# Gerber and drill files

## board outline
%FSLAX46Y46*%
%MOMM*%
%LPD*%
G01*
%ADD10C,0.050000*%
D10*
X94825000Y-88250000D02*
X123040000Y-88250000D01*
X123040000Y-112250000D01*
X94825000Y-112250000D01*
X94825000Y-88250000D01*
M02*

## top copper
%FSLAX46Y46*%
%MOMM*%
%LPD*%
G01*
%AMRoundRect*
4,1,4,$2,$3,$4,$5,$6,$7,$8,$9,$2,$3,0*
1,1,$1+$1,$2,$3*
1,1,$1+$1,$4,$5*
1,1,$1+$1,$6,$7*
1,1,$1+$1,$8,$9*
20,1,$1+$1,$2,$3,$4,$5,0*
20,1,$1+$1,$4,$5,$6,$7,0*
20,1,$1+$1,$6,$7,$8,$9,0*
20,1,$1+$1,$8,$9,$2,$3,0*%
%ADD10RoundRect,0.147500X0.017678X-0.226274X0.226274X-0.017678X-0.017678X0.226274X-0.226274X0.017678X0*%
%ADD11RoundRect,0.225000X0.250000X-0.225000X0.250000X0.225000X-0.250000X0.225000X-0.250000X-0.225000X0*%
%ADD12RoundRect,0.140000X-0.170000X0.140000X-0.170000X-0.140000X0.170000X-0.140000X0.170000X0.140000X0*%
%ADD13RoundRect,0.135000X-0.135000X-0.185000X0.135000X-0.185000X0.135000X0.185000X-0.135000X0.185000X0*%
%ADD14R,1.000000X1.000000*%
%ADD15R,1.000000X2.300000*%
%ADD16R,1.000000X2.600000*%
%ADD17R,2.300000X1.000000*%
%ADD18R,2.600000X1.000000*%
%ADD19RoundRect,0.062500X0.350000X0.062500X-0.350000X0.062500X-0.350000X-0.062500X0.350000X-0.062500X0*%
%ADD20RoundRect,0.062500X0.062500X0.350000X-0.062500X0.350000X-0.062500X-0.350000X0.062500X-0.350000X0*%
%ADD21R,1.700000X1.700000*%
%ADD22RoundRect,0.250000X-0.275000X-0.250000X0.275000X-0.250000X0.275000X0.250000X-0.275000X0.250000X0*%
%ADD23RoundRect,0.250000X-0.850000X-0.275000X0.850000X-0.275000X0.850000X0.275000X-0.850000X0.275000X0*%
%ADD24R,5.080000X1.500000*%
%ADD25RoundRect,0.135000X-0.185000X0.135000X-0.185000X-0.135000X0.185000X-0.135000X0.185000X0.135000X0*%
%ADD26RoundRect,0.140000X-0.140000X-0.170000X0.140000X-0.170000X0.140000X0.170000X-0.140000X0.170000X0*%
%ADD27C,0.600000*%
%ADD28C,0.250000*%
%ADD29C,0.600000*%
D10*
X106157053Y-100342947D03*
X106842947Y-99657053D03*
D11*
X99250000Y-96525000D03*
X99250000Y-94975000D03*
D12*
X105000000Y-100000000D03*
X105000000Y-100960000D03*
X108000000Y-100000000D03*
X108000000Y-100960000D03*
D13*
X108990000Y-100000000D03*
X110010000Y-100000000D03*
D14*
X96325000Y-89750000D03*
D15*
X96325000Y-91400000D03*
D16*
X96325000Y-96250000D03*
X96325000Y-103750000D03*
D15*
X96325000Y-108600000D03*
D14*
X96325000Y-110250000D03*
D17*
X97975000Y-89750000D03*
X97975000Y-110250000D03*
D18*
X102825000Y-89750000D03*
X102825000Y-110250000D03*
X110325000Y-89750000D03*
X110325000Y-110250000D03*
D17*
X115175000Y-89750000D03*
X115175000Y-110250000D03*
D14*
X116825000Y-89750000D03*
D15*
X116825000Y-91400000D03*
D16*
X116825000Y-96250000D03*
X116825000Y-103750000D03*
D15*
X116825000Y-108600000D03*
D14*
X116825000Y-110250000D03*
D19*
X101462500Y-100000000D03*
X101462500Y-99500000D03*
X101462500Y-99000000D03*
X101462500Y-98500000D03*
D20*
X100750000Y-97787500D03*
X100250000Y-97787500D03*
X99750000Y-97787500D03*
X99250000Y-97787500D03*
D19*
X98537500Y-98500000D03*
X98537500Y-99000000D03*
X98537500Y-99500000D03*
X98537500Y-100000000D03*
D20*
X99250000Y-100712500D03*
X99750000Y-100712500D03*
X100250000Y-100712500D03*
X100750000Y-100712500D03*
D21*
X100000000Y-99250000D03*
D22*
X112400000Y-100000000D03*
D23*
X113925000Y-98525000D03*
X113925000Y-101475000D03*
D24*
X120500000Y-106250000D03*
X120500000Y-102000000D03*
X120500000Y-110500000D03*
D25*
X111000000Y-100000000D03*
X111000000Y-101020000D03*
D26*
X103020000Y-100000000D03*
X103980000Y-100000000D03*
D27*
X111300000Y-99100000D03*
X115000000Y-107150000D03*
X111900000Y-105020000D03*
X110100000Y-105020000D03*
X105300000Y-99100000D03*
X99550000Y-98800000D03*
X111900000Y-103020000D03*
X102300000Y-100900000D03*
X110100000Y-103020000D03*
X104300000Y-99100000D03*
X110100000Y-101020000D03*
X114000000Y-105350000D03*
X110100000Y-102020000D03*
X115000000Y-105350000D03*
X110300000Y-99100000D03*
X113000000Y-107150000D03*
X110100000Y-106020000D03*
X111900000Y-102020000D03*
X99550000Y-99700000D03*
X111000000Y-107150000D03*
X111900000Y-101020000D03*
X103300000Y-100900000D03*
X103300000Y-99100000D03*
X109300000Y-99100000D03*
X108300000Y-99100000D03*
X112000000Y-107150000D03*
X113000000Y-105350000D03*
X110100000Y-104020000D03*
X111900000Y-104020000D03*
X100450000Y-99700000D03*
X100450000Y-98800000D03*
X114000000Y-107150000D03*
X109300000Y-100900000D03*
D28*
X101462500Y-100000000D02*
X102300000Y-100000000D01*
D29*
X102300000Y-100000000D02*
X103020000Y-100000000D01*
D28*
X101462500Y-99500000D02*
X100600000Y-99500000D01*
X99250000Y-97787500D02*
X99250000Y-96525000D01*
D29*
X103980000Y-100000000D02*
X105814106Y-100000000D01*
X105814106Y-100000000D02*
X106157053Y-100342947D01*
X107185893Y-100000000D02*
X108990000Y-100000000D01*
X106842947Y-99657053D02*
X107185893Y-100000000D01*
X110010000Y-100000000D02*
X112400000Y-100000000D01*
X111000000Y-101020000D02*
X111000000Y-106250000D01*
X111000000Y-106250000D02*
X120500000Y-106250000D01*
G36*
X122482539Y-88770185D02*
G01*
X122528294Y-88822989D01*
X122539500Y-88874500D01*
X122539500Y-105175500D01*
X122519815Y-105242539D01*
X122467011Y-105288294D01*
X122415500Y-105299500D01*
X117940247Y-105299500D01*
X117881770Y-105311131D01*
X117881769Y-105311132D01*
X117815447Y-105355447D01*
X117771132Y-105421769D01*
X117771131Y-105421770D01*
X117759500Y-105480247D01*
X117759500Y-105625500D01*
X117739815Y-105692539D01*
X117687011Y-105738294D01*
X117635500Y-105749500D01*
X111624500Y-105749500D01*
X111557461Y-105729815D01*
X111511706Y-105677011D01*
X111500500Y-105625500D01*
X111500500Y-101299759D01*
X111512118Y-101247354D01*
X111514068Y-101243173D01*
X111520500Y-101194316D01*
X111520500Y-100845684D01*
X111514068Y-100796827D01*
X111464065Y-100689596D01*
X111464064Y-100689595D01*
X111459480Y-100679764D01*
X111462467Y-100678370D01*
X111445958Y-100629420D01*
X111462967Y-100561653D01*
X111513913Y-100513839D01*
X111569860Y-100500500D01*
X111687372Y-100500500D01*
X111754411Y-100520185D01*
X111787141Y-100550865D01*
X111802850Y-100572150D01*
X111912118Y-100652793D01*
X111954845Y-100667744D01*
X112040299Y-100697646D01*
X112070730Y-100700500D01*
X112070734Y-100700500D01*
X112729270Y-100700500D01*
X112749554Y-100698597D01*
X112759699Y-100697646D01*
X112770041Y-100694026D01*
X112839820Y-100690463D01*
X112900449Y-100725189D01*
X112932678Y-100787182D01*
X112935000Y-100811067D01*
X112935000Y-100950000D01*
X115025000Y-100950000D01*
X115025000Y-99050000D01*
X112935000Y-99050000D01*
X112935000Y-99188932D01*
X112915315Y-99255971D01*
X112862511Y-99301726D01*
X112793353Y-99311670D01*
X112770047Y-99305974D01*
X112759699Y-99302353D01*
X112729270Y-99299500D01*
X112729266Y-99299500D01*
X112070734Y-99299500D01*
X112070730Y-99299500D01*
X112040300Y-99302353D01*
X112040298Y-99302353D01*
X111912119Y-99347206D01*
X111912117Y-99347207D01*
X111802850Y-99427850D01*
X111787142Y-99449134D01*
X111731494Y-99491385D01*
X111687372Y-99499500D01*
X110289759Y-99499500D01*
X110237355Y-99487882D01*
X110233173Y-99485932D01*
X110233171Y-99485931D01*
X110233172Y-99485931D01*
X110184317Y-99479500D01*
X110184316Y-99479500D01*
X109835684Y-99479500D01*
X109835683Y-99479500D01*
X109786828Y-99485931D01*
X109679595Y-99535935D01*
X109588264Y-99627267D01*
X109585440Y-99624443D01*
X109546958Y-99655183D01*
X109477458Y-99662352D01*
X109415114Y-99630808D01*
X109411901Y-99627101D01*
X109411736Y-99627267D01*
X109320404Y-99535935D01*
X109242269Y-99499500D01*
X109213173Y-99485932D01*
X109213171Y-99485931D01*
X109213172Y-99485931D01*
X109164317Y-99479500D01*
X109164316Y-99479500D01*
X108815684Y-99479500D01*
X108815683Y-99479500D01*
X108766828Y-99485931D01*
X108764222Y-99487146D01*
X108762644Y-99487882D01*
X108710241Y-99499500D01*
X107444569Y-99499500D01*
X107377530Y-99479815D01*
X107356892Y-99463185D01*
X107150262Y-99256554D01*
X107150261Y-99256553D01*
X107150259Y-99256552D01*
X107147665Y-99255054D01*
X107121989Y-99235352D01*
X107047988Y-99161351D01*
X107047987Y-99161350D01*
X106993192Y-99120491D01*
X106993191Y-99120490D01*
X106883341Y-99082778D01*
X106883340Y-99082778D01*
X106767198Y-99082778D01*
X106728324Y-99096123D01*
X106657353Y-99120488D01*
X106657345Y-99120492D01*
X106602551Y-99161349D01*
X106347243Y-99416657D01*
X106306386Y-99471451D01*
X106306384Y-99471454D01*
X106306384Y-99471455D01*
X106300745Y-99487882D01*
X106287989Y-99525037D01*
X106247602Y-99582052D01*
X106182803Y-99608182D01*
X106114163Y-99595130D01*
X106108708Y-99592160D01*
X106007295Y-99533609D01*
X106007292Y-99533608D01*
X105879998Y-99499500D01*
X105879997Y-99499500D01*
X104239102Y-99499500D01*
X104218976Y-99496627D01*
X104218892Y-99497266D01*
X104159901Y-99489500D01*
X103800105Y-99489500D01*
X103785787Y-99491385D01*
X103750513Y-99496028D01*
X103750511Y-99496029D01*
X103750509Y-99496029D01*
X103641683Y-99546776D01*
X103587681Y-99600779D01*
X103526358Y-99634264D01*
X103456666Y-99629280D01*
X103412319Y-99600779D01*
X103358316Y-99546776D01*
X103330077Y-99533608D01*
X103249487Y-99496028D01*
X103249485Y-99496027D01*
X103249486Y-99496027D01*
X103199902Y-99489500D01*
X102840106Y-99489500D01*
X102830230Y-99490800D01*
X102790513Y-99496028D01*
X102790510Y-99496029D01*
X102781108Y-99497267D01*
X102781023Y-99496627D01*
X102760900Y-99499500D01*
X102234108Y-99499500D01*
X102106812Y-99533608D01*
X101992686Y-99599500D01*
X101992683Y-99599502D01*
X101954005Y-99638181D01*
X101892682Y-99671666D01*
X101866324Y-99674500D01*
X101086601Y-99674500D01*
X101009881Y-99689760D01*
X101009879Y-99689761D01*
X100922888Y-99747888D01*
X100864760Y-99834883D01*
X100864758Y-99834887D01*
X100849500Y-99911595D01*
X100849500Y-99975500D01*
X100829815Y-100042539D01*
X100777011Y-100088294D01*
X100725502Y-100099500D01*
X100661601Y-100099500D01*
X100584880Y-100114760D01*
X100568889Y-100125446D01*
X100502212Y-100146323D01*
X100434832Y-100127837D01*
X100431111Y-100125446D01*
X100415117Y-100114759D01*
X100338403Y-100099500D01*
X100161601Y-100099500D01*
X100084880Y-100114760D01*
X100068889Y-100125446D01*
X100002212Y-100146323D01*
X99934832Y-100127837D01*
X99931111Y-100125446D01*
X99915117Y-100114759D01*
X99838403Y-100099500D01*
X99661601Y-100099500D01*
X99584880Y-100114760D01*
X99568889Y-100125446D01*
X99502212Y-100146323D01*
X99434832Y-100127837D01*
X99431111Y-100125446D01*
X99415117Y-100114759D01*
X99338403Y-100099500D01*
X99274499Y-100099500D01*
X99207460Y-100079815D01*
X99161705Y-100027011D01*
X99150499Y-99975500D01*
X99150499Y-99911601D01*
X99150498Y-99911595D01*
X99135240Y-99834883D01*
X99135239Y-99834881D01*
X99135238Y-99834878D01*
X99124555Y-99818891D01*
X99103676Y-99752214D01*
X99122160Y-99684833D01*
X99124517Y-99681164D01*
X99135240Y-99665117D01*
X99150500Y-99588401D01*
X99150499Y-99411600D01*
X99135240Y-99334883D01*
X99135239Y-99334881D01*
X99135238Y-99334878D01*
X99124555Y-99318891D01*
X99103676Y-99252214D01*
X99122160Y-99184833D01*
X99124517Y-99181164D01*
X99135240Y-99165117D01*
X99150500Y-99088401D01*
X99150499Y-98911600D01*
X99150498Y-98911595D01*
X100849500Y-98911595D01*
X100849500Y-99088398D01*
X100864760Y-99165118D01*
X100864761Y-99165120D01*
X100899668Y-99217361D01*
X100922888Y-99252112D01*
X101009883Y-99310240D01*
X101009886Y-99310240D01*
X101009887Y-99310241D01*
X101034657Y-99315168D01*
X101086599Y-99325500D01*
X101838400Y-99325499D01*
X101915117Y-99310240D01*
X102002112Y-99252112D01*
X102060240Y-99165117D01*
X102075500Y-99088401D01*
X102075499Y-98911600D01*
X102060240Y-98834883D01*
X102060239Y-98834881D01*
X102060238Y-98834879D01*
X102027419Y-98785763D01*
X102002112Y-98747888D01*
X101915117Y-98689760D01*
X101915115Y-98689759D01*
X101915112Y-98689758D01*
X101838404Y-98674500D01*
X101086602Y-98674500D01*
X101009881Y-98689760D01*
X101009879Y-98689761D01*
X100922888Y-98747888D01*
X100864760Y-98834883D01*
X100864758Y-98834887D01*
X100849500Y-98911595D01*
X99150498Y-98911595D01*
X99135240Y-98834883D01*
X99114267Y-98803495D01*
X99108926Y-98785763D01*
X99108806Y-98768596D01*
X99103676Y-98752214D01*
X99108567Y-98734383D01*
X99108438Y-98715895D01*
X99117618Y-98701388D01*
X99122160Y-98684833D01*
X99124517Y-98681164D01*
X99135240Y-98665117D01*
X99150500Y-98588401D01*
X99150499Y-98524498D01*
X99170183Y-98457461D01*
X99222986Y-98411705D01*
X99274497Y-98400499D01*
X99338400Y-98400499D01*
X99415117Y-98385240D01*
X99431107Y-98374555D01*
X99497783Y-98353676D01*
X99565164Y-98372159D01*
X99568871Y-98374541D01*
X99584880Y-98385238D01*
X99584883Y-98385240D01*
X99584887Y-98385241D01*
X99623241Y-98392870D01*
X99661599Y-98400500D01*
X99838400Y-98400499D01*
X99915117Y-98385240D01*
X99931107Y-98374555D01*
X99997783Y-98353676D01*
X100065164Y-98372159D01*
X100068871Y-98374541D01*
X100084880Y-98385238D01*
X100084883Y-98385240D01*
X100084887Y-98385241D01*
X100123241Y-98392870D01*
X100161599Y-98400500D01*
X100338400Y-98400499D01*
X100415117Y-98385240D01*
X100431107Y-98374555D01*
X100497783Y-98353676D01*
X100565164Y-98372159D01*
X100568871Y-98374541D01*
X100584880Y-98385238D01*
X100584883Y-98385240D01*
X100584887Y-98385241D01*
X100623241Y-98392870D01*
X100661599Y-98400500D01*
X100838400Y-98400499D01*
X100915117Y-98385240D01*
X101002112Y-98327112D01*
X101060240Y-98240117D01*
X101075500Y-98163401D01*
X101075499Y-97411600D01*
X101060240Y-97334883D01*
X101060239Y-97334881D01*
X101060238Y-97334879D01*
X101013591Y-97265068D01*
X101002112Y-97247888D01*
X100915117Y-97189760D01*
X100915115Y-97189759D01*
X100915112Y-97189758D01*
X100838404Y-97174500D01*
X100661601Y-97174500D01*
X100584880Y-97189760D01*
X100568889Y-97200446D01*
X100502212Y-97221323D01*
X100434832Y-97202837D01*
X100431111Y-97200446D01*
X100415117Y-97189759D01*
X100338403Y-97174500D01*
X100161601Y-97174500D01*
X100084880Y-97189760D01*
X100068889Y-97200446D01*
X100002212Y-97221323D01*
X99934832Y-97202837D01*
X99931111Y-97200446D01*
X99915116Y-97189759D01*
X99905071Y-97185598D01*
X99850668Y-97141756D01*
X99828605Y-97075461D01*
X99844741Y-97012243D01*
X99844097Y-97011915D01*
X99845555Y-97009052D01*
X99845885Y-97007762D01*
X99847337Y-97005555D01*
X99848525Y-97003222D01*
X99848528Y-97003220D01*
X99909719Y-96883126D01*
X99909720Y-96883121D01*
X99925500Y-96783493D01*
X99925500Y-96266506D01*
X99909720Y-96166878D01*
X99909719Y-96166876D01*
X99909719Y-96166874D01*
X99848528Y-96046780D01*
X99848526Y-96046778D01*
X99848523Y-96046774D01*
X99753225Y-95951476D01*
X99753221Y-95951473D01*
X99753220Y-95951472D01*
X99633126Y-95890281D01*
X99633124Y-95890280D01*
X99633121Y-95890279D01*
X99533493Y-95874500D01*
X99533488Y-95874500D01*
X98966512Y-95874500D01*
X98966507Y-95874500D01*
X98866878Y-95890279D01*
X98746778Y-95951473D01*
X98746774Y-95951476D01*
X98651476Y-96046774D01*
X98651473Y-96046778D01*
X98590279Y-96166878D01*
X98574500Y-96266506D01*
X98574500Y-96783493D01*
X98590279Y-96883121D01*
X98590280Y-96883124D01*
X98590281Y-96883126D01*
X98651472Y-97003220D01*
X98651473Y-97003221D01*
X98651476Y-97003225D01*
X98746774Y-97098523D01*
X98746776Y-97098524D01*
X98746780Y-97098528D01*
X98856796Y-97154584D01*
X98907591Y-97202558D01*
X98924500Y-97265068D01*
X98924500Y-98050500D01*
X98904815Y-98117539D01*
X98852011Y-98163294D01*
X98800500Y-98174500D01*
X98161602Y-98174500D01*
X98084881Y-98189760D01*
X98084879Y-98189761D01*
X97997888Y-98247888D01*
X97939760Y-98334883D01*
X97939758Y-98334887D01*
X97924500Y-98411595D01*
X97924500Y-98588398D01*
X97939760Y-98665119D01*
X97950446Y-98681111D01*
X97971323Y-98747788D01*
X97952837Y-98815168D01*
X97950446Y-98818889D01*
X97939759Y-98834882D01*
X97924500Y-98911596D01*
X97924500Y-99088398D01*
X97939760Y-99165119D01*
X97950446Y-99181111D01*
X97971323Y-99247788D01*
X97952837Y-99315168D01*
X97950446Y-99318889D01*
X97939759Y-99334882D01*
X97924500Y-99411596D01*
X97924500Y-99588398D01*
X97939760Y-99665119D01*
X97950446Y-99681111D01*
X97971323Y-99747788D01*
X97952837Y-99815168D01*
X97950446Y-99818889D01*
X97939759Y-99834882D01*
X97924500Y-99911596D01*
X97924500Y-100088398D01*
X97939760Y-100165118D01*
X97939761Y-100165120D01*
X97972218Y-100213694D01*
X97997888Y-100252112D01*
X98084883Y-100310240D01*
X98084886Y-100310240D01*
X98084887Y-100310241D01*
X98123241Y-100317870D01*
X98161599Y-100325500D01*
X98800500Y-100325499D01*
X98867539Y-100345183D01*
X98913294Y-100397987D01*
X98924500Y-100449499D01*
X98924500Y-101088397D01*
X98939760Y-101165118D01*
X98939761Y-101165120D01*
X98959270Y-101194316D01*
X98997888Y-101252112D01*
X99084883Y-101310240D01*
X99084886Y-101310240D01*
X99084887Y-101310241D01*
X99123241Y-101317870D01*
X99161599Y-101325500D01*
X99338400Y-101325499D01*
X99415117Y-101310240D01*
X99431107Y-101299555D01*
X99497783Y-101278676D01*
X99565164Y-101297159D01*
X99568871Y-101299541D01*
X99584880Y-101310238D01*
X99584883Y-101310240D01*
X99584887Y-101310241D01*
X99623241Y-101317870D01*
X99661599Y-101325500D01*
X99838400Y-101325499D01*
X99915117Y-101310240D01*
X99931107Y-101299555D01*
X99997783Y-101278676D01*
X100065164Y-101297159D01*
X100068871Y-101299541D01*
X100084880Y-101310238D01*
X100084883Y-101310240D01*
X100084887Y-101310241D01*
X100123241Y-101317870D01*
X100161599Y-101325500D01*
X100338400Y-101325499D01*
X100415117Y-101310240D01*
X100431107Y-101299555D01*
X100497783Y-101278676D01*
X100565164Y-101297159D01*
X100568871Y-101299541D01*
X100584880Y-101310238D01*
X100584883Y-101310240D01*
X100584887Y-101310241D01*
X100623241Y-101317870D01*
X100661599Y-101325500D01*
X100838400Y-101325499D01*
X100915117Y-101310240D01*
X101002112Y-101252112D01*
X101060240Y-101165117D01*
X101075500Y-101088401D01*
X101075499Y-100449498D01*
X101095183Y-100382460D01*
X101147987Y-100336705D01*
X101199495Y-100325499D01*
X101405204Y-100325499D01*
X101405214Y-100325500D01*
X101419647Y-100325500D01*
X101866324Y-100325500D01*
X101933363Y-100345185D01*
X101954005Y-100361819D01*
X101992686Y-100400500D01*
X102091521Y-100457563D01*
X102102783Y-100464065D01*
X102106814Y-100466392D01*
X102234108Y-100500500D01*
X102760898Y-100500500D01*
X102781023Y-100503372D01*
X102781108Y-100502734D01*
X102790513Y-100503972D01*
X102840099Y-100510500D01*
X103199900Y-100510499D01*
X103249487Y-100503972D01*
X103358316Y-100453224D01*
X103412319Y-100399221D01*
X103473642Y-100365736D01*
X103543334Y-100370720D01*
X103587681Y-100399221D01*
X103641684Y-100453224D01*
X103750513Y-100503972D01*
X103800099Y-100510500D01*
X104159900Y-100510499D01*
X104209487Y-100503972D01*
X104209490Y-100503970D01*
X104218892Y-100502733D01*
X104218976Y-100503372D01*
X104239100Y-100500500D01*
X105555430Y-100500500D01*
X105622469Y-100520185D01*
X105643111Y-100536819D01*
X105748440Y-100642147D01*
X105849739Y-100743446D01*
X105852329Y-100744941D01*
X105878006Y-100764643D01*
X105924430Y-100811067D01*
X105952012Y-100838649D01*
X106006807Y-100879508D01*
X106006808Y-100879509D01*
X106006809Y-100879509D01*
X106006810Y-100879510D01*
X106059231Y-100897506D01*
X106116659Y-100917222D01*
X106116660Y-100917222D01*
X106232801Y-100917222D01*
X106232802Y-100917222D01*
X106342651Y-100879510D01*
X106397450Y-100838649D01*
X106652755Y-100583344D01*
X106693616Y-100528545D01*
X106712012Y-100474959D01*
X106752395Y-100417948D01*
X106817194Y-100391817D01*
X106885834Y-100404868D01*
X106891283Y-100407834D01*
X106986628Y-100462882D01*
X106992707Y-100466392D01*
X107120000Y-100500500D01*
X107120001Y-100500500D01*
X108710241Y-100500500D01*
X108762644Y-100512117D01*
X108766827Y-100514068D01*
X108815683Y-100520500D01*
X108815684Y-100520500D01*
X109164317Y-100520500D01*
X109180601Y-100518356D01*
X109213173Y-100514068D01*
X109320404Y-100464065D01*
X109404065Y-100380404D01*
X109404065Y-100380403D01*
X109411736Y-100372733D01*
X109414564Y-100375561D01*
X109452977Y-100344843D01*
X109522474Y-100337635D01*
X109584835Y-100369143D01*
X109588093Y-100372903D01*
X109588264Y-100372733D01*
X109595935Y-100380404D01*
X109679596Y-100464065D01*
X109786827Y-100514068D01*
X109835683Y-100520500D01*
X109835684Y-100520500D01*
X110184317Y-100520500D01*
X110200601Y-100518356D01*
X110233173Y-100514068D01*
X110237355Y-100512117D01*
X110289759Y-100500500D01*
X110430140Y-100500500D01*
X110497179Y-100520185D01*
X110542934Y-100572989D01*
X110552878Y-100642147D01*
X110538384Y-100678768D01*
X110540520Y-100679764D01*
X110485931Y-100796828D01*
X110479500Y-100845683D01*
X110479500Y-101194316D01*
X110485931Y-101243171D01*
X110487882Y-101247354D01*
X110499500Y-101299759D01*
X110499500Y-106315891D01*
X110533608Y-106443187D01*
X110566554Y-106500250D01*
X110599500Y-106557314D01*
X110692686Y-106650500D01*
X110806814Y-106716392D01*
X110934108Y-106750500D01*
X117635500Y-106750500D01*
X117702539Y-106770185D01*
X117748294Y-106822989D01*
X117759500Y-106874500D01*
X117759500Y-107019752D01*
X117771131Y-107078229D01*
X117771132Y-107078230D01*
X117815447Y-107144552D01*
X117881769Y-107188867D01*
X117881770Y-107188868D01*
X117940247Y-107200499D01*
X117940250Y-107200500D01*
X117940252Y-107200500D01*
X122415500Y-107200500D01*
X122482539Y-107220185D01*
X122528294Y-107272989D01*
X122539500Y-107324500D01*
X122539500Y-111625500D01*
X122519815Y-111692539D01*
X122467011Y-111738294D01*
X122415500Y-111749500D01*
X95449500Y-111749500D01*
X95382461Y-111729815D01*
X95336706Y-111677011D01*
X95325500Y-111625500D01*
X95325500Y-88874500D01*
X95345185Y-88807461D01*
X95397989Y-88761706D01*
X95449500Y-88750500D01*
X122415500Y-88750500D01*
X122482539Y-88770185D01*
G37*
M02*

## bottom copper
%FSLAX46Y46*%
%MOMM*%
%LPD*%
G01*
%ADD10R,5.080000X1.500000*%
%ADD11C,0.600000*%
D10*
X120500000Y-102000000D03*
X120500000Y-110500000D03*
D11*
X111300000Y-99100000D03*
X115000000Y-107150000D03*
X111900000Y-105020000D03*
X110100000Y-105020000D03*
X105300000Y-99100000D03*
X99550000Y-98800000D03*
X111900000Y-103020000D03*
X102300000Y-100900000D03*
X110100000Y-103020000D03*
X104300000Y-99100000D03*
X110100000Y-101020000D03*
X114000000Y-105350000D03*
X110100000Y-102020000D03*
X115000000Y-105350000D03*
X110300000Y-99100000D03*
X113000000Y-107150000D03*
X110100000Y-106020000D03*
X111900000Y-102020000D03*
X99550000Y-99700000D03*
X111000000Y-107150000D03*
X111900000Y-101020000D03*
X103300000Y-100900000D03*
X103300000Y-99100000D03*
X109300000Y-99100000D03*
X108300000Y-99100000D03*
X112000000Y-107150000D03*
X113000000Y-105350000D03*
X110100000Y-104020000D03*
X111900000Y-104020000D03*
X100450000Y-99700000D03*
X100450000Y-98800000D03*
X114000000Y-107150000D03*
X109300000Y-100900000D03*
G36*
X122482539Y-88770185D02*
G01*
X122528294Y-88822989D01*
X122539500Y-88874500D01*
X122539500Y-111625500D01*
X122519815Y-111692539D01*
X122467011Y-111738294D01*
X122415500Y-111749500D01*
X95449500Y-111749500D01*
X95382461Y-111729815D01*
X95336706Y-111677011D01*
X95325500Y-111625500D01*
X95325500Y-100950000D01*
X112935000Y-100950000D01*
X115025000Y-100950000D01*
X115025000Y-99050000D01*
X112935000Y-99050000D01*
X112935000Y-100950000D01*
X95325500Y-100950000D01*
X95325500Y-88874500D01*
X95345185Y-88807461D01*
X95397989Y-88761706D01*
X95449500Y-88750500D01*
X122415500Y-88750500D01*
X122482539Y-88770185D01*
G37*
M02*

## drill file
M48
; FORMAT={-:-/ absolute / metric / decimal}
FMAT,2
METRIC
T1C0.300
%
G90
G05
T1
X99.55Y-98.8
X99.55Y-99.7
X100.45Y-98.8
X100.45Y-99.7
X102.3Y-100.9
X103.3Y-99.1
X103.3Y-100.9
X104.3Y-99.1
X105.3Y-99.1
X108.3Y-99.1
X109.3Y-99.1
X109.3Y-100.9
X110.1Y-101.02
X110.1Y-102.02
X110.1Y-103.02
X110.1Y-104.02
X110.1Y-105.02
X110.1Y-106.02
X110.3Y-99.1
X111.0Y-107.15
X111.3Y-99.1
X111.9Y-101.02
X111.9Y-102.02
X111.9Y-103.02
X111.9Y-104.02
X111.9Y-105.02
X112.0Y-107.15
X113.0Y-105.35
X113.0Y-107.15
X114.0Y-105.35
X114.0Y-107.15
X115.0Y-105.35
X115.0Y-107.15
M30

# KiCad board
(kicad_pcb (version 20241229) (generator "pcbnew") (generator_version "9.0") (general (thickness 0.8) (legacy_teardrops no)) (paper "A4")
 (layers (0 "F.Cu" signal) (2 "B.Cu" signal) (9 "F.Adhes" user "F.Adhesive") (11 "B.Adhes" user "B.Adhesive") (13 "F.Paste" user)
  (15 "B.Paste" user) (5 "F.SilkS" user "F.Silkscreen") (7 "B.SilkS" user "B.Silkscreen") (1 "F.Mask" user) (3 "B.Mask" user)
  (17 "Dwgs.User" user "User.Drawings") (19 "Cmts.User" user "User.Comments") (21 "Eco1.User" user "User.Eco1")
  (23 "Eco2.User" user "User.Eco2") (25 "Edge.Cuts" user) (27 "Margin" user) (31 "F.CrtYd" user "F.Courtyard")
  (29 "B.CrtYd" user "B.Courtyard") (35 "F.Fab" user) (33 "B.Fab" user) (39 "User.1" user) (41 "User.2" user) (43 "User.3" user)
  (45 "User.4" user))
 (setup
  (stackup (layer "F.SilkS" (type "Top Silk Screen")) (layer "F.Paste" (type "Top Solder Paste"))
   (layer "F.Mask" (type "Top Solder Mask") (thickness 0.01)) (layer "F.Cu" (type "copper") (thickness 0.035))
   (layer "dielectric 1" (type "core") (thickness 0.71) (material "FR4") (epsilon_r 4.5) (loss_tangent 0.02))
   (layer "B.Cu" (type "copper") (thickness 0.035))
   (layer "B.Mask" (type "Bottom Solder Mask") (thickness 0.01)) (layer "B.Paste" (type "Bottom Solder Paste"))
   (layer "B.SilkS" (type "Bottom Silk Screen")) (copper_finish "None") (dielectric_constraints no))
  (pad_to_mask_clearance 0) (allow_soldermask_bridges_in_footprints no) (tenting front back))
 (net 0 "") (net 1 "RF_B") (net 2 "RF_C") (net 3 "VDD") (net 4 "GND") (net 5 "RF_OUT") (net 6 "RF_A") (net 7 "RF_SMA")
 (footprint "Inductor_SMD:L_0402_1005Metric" (layer "F.Cu") (at 106.5 100 45)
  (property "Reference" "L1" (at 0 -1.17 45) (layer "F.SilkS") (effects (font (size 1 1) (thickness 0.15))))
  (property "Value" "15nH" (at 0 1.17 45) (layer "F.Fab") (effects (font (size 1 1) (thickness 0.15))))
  (pad "1" smd roundrect (at -0.485 0 45) (size 0.59 0.64) (layers "F.Cu" "F.Mask" "F.Paste") (roundrect_rratio 0.25) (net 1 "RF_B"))
  (pad "2" smd roundrect (at 0.485 0 45) (size 0.59 0.64) (layers "F.Cu" "F.Mask" "F.Paste") (roundrect_rratio 0.25) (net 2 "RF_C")))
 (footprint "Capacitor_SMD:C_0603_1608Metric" (layer "F.Cu") (at 99.25 95.75 90)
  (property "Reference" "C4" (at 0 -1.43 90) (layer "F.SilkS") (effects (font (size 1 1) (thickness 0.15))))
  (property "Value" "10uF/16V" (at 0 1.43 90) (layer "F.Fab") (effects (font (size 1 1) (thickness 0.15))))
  (pad "1" smd roundrect (at -0.775 0 90) (size 0.9 0.95) (layers "F.Cu" "F.Mask" "F.Paste") (roundrect_rratio 0.25) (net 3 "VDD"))
  (pad "2" smd roundrect (at 0.775 0 90) (size 0.9 0.95) (layers "F.Cu" "F.Mask" "F.Paste") (roundrect_rratio 0.25) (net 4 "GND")))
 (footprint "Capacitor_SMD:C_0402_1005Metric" (layer "F.Cu") (at 105 100.48 -90)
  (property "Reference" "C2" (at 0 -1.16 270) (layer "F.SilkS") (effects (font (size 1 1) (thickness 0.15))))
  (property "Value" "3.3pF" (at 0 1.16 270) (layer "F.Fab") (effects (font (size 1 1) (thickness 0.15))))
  (pad "1" smd roundrect (at -0.48 0 270) (size 0.56 0.62) (layers "F.Cu" "F.Mask" "F.Paste") (roundrect_rratio 0.25) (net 1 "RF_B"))
  (pad "2" smd roundrect (at 0.48 0 270) (size 0.56 0.62) (layers "F.Cu" "F.Mask" "F.Paste") (roundrect_rratio 0.25) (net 4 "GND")))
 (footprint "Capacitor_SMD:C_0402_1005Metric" (layer "F.Cu") (at 108 100.48 -90)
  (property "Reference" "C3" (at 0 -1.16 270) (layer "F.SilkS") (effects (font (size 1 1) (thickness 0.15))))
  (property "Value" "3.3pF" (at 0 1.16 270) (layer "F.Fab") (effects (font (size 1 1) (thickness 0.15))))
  (pad "1" smd roundrect (at -0.48 0 270) (size 0.56 0.62) (layers "F.Cu" "F.Mask" "F.Paste") (roundrect_rratio 0.25) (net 2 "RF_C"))
  (pad "2" smd roundrect (at 0.48 0 270) (size 0.56 0.62) (layers "F.Cu" "F.Mask" "F.Paste") (roundrect_rratio 0.25) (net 4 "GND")))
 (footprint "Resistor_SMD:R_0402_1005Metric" (layer "F.Cu") (at 109.5 100)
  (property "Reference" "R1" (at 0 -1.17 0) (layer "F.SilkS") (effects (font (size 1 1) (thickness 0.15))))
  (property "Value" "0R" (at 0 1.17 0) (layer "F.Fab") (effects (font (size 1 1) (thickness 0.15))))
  (pad "1" smd roundrect (at -0.51 0) (size 0.54 0.64) (layers "F.Cu" "F.Mask" "F.Paste") (roundrect_rratio 0.25) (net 2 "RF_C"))
  (pad "2" smd roundrect (at 0.51 0) (size 0.54 0.64) (layers "F.Cu" "F.Mask" "F.Paste") (roundrect_rratio 0.25) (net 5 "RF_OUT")))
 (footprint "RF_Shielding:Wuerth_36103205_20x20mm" (layer "F.Cu") (at 106.575 100)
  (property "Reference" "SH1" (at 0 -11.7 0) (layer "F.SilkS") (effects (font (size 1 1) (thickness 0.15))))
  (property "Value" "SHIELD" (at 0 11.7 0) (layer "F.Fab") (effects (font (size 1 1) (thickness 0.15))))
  (pad "1" smd rect (at -10.25 -10.25) (size 1 1) (layers "F.Cu" "F.Mask" "F.Paste") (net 4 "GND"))
  (pad "1" smd rect (at -10.25 -8.6) (size 1 2.3) (layers "F.Cu" "F.Mask" "F.Paste") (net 4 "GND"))
  (pad "1" smd rect (at -10.25 -3.75) (size 1 2.6) (layers "F.Cu" "F.Mask" "F.Paste") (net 4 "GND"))
  (pad "1" smd rect (at -10.25 3.75) (size 1 2.6) (layers "F.Cu" "F.Mask" "F.Paste") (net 4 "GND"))
  (pad "1" smd rect (at -10.25 8.6) (size 1 2.3) (layers "F.Cu" "F.Mask" "F.Paste") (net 4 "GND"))
  (pad "1" smd rect (at -10.25 10.25) (size 1 1) (layers "F.Cu" "F.Mask" "F.Paste") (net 4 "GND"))
  (pad "1" smd rect (at -8.6 -10.25) (size 2.3 1) (layers "F.Cu" "F.Mask" "F.Paste") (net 4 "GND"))
  (pad "1" smd rect (at -8.6 10.25) (size 2.3 1) (layers "F.Cu" "F.Mask" "F.Paste") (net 4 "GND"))
  (pad "1" smd rect (at -3.75 -10.25) (size 2.6 1) (layers "F.Cu" "F.Mask" "F.Paste") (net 4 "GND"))
  (pad "1" smd rect (at -3.75 10.25) (size 2.6 1) (layers "F.Cu" "F.Mask" "F.Paste") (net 4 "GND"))
  (pad "1" smd rect (at 3.75 -10.25) (size 2.6 1) (layers "F.Cu" "F.Mask" "F.Paste") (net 4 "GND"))
  (pad "1" smd rect (at 3.75 10.25) (size 2.6 1) (layers "F.Cu" "F.Mask" "F.Paste") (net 4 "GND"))
  (pad "1" smd rect (at 8.6 -10.25) (size 2.3 1) (layers "F.Cu" "F.Mask" "F.Paste") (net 4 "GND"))
  (pad "1" smd rect (at 8.6 10.25) (size 2.3 1) (layers "F.Cu" "F.Mask" "F.Paste") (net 4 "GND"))
  (pad "1" smd rect (at 10.25 -10.25) (size 1 1) (layers "F.Cu" "F.Mask" "F.Paste") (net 4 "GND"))
  (pad "1" smd rect (at 10.25 -8.6) (size 1 2.3) (layers "F.Cu" "F.Mask" "F.Paste") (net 4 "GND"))
  (pad "1" smd rect (at 10.25 -3.75) (size 1 2.6) (layers "F.Cu" "F.Mask" "F.Paste") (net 4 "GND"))
  (pad "1" smd rect (at 10.25 3.75) (size 1 2.6) (layers "F.Cu" "F.Mask" "F.Paste") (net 4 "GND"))
  (pad "1" smd rect (at 10.25 8.6) (size 1 2.3) (layers "F.Cu" "F.Mask" "F.Paste") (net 4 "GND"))
  (pad "1" smd rect (at 10.25 10.25) (size 1 1) (layers "F.Cu" "F.Mask" "F.Paste") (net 4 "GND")))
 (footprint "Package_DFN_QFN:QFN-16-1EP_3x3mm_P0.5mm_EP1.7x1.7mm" (layer "F.Cu") (at 100 99.25 180)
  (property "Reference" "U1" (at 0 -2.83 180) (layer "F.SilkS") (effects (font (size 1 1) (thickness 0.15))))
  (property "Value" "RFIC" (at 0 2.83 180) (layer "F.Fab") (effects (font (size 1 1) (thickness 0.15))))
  (pad "" smd roundrect (at -0.425 -0.425 180) (size 0.69 0.69) (layers "F.Paste") (roundrect_rratio 0.25))
  (pad "" smd roundrect (at -0.425 0.425 180) (size 0.69 0.69) (layers "F.Paste") (roundrect_rratio 0.25))
  (pad "" smd roundrect (at 0.425 -0.425 180) (size 0.69 0.69) (layers "F.Paste") (roundrect_rratio 0.25))
  (pad "" smd roundrect (at 0.425 0.425 180) (size 0.69 0.69) (layers "F.Paste") (roundrect_rratio 0.25))
  (pad "1" smd roundrect (at -1.4625 -0.75 180) (size 0.825 0.25) (layers "F.Cu" "F.Mask" "F.Paste") (roundrect_rratio 0.25) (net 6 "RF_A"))
  (pad "2" smd roundrect (at -1.4625 -0.25 180) (size 0.825 0.25) (layers "F.Cu" "F.Mask" "F.Paste") (roundrect_rratio 0.25) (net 4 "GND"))
  (pad "3" smd roundrect (at -1.4625 0.25 180) (size 0.825 0.25) (layers "F.Cu" "F.Mask" "F.Paste") (roundrect_rratio 0.25))
  (pad "4" smd roundrect (at -1.4625 0.75 180) (size 0.825 0.25) (layers "F.Cu" "F.Mask" "F.Paste") (roundrect_rratio 0.25) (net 4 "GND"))
  (pad "5" smd roundrect (at -0.75 1.4625 180) (size 0.25 0.825) (layers "F.Cu" "F.Mask" "F.Paste") (roundrect_rratio 0.25))
  (pad "6" smd roundrect (at -0.25 1.4625 180) (size 0.25 0.825) (layers "F.Cu" "F.Mask" "F.Paste") (roundrect_rratio 0.25))
  (pad "7" smd roundrect (at 0.25 1.4625 180) (size 0.25 0.825) (layers "F.Cu" "F.Mask" "F.Paste") (roundrect_rratio 0.25))
  (pad "8" smd roundrect (at 0.75 1.4625 180) (size 0.25 0.825) (layers "F.Cu" "F.Mask" "F.Paste") (roundrect_rratio 0.25) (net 3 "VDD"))
  (pad "9" smd roundrect (at 1.4625 0.75 180) (size 0.825 0.25) (layers "F.Cu" "F.Mask" "F.Paste") (roundrect_rratio 0.25))
  (pad "10" smd roundrect (at 1.4625 0.25 180) (size 0.825 0.25) (layers "F.Cu" "F.Mask" "F.Paste") (roundrect_rratio 0.25))
  (pad "11" smd roundrect (at 1.4625 -0.25 180) (size 0.825 0.25) (layers "F.Cu" "F.Mask" "F.Paste") (roundrect_rratio 0.25))
  (pad "12" smd roundrect (at 1.4625 -0.75 180) (size 0.825 0.25) (layers "F.Cu" "F.Mask" "F.Paste") (roundrect_rratio 0.25))
  (pad "13" smd roundrect (at 0.75 -1.4625 180) (size 0.25 0.825) (layers "F.Cu" "F.Mask" "F.Paste") (roundrect_rratio 0.25))
  (pad "14" smd roundrect (at 0.25 -1.4625 180) (size 0.25 0.825) (layers "F.Cu" "F.Mask" "F.Paste") (roundrect_rratio 0.25))
  (pad "15" smd roundrect (at -0.25 -1.4625 180) (size 0.25 0.825) (layers "F.Cu" "F.Mask" "F.Paste") (roundrect_rratio 0.25))
  (pad "16" smd roundrect (at -0.75 -1.4625 180) (size 0.25 0.825) (layers "F.Cu" "F.Mask" "F.Paste") (roundrect_rratio 0.25))
  (pad "17" smd rect (at 0 0 180) (size 1.7 1.7) (layers "F.Cu" "F.Mask") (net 4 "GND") (zone_connect 2)))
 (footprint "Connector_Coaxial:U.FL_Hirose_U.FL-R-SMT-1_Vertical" (layer "F.Cu") (at 113.45 100)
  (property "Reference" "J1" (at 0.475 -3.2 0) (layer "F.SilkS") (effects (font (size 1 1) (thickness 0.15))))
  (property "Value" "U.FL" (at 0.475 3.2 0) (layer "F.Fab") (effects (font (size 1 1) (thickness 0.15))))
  (pad "1" smd roundrect (at -1.05 0) (size 1.05 1) (layers "F.Cu" "F.Mask" "F.Paste") (roundrect_rratio 0.25) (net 5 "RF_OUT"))
  (pad "2" smd roundrect (at 0.475 -1.475) (size 2.2 1.05) (layers "F.Cu" "F.Mask" "F.Paste") (roundrect_rratio 0.2380952381) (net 4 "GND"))
  (pad "2" smd roundrect (at 0.475 1.475) (size 2.2 1.05) (layers "F.Cu" "F.Mask" "F.Paste") (roundrect_rratio 0.2380952381) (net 4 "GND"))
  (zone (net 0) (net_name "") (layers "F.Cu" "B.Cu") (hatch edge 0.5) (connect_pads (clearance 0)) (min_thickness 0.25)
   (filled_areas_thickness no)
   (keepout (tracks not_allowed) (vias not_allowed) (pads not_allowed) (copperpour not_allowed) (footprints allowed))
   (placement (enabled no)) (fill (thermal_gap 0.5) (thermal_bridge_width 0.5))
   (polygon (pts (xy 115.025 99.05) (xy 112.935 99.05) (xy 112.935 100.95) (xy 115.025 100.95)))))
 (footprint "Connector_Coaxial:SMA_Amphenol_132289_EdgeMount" (layer "F.Cu") (at 120.5 106.25)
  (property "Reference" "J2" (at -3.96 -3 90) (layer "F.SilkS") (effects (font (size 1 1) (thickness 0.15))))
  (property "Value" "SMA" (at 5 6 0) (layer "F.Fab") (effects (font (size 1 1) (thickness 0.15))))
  (pad "1" smd rect (at 0 0 90) (size 1.5 5.08) (layers "F.Cu" "F.Mask" "F.Paste") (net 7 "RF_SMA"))
  (pad "2" smd rect (at 0 -4.25 90) (size 1.5 5.08) (layers "F.Cu" "F.Mask" "F.Paste") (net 4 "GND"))
  (pad "2" smd rect (at 0 -4.25 90) (size 1.5 5.08) (layers "B.Cu" "B.Mask" "B.Paste") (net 4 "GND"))
  (pad "2" smd rect (at 0 4.25 90) (size 1.5 5.08) (layers "F.Cu" "F.Mask" "F.Paste") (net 4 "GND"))
  (pad "2" smd rect (at 0 4.25 90) (size 1.5 5.08) (layers "B.Cu" "B.Mask" "B.Paste") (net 4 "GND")))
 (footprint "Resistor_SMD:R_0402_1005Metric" (layer "F.Cu") (at 111 100.51 -90)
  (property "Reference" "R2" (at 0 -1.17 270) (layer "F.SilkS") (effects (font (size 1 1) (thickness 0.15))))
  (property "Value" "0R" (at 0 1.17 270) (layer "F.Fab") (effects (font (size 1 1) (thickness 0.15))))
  (pad "1" smd roundrect (at -0.51 0 270) (size 0.54 0.64) (layers "F.Cu" "F.Mask" "F.Paste") (roundrect_rratio 0.25) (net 5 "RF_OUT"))
  (pad "2" smd roundrect (at 0.51 0 270) (size 0.54 0.64) (layers "F.Cu" "F.Mask" "F.Paste") (roundrect_rratio 0.25) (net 7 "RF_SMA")))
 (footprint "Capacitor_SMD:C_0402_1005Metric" (layer "F.Cu") (at 103.5 100)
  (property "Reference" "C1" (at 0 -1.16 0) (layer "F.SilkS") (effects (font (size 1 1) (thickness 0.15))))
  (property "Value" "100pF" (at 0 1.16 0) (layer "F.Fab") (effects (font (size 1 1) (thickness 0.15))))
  (pad "1" smd roundrect (at -0.48 0) (size 0.56 0.62) (layers "F.Cu" "F.Mask" "F.Paste") (roundrect_rratio 0.25) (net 6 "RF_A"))
  (pad "2" smd roundrect (at 0.48 0) (size 0.56 0.62) (layers "F.Cu" "F.Mask" "F.Paste") (roundrect_rratio 0.25) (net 1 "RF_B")))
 (gr_rect (start 94.825 88.25) (end 123.04 112.25) (stroke (width 0.05) (type default)) (fill no) (layer "Edge.Cuts"))
 (segment (start 101.4625 100) (end 102.3 100) (width 0.25) (layer "F.Cu") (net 6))
 (segment (start 102.3 100) (end 103.02 100) (width 0.6) (layer "F.Cu") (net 6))
 (segment (start 101.4625 99.5) (end 100.6 99.5) (width 0.25) (layer "F.Cu") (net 4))
 (via (at 111.3 99.1) (size 0.6) (drill 0.3) (layers "F.Cu" "B.Cu") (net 4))
 (via (at 115 107.15) (size 0.6) (drill 0.3) (layers "F.Cu" "B.Cu") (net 4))
 (via (at 111.9 105.02) (size 0.6) (drill 0.3) (layers "F.Cu" "B.Cu") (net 4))
 (via (at 110.1 105.02) (size 0.6) (drill 0.3) (layers "F.Cu" "B.Cu") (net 4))
 (via (at 105.3 99.1) (size 0.6) (drill 0.3) (layers "F.Cu" "B.Cu") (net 4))
 (via (at 99.55 98.8) (size 0.6) (drill 0.3) (layers "F.Cu" "B.Cu") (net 4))
 (via (at 111.9 103.02) (size 0.6) (drill 0.3) (layers "F.Cu" "B.Cu") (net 4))
 (via (at 102.3 100.9) (size 0.6) (drill 0.3) (layers "F.Cu" "B.Cu") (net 4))
 (via (at 110.1 103.02) (size 0.6) (drill 0.3) (layers "F.Cu" "B.Cu") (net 4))
 (via (at 104.3 99.1) (size 0.6) (drill 0.3) (layers "F.Cu" "B.Cu") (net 4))
 (via (at 110.1 101.02) (size 0.6) (drill 0.3) (layers "F.Cu" "B.Cu") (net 4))
 (via (at 114 105.35) (size 0.6) (drill 0.3) (layers "F.Cu" "B.Cu") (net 4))
 (via (at 110.1 102.02) (size 0.6) (drill 0.3) (layers "F.Cu" "B.Cu") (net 4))
 (via (at 115 105.35) (size 0.6) (drill 0.3) (layers "F.Cu" "B.Cu") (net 4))
 (via (at 110.3 99.1) (size 0.6) (drill 0.3) (layers "F.Cu" "B.Cu") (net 4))
 (via (at 113 107.15) (size 0.6) (drill 0.3) (layers "F.Cu" "B.Cu") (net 4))
 (via (at 110.1 106.02) (size 0.6) (drill 0.3) (layers "F.Cu" "B.Cu") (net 4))
 (via (at 111.9 102.02) (size 0.6) (drill 0.3) (layers "F.Cu" "B.Cu") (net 4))
 (via (at 99.55 99.7) (size 0.6) (drill 0.3) (layers "F.Cu" "B.Cu") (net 4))
 (via (at 111 107.15) (size 0.6) (drill 0.3) (layers "F.Cu" "B.Cu") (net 4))
 (via (at 111.9 101.02) (size 0.6) (drill 0.3) (layers "F.Cu" "B.Cu") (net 4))
 (via (at 103.3 100.9) (size 0.6) (drill 0.3) (layers "F.Cu" "B.Cu") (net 4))
 (via (at 103.3 99.1) (size 0.6) (drill 0.3) (layers "F.Cu" "B.Cu") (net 4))
 (via (at 109.3 99.1) (size 0.6) (drill 0.3) (layers "F.Cu" "B.Cu") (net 4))
 (via (at 108.3 99.1) (size 0.6) (drill 0.3) (layers "F.Cu" "B.Cu") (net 4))
 (via (at 112 107.15) (size 0.6) (drill 0.3) (layers "F.Cu" "B.Cu") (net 4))
 (via (at 113 105.35) (size 0.6) (drill 0.3) (layers "F.Cu" "B.Cu") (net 4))
 (via (at 110.1 104.02) (size 0.6) (drill 0.3) (layers "F.Cu" "B.Cu") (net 4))
 (via (at 111.9 104.02) (size 0.6) (drill 0.3) (layers "F.Cu" "B.Cu") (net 4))
 (via (at 100.45 99.7) (size 0.6) (drill 0.3) (layers "F.Cu" "B.Cu") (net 4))
 (via (at 100.45 98.8) (size 0.6) (drill 0.3) (layers "F.Cu" "B.Cu") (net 4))
 (via (at 114 107.15) (size 0.6) (drill 0.3) (layers "F.Cu" "B.Cu") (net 4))
 (via (at 109.3 100.9) (size 0.6) (drill 0.3) (layers "F.Cu" "B.Cu") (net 4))
 (segment (start 99.25 97.7875) (end 99.25 96.525) (width 0.25) (layer "F.Cu") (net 3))
 (segment (start 103.98 100) (end 105.814106 100) (width 0.6) (layer "F.Cu") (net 1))
 (segment (start 105.814106 100) (end 106.157053 100.342947) (width 0.6) (layer "F.Cu") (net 1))
 (segment (start 107.185893 100) (end 108.99 100) (width 0.6) (layer "F.Cu") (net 2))
 (segment (start 106.842947 99.657053) (end 107.185893 100) (width 0.6) (layer "F.Cu") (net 2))
 (segment (start 110.01 100) (end 112.4 100) (width 0.6) (layer "F.Cu") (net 5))
 (segment (start 111 101.02) (end 111 106.25) (width 0.6) (layer "F.Cu") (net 7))
 (segment (start 111 106.25) (end 120.5 106.25) (width 0.6) (layer "F.Cu") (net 7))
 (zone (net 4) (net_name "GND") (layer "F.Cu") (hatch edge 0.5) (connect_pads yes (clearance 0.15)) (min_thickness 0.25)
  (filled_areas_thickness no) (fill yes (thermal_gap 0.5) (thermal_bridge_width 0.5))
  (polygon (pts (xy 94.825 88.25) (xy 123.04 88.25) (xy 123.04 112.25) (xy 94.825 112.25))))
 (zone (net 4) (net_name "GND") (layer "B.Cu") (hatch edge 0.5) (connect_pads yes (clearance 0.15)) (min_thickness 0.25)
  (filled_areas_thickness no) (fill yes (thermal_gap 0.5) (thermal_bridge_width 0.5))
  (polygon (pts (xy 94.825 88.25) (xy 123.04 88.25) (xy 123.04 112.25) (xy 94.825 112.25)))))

